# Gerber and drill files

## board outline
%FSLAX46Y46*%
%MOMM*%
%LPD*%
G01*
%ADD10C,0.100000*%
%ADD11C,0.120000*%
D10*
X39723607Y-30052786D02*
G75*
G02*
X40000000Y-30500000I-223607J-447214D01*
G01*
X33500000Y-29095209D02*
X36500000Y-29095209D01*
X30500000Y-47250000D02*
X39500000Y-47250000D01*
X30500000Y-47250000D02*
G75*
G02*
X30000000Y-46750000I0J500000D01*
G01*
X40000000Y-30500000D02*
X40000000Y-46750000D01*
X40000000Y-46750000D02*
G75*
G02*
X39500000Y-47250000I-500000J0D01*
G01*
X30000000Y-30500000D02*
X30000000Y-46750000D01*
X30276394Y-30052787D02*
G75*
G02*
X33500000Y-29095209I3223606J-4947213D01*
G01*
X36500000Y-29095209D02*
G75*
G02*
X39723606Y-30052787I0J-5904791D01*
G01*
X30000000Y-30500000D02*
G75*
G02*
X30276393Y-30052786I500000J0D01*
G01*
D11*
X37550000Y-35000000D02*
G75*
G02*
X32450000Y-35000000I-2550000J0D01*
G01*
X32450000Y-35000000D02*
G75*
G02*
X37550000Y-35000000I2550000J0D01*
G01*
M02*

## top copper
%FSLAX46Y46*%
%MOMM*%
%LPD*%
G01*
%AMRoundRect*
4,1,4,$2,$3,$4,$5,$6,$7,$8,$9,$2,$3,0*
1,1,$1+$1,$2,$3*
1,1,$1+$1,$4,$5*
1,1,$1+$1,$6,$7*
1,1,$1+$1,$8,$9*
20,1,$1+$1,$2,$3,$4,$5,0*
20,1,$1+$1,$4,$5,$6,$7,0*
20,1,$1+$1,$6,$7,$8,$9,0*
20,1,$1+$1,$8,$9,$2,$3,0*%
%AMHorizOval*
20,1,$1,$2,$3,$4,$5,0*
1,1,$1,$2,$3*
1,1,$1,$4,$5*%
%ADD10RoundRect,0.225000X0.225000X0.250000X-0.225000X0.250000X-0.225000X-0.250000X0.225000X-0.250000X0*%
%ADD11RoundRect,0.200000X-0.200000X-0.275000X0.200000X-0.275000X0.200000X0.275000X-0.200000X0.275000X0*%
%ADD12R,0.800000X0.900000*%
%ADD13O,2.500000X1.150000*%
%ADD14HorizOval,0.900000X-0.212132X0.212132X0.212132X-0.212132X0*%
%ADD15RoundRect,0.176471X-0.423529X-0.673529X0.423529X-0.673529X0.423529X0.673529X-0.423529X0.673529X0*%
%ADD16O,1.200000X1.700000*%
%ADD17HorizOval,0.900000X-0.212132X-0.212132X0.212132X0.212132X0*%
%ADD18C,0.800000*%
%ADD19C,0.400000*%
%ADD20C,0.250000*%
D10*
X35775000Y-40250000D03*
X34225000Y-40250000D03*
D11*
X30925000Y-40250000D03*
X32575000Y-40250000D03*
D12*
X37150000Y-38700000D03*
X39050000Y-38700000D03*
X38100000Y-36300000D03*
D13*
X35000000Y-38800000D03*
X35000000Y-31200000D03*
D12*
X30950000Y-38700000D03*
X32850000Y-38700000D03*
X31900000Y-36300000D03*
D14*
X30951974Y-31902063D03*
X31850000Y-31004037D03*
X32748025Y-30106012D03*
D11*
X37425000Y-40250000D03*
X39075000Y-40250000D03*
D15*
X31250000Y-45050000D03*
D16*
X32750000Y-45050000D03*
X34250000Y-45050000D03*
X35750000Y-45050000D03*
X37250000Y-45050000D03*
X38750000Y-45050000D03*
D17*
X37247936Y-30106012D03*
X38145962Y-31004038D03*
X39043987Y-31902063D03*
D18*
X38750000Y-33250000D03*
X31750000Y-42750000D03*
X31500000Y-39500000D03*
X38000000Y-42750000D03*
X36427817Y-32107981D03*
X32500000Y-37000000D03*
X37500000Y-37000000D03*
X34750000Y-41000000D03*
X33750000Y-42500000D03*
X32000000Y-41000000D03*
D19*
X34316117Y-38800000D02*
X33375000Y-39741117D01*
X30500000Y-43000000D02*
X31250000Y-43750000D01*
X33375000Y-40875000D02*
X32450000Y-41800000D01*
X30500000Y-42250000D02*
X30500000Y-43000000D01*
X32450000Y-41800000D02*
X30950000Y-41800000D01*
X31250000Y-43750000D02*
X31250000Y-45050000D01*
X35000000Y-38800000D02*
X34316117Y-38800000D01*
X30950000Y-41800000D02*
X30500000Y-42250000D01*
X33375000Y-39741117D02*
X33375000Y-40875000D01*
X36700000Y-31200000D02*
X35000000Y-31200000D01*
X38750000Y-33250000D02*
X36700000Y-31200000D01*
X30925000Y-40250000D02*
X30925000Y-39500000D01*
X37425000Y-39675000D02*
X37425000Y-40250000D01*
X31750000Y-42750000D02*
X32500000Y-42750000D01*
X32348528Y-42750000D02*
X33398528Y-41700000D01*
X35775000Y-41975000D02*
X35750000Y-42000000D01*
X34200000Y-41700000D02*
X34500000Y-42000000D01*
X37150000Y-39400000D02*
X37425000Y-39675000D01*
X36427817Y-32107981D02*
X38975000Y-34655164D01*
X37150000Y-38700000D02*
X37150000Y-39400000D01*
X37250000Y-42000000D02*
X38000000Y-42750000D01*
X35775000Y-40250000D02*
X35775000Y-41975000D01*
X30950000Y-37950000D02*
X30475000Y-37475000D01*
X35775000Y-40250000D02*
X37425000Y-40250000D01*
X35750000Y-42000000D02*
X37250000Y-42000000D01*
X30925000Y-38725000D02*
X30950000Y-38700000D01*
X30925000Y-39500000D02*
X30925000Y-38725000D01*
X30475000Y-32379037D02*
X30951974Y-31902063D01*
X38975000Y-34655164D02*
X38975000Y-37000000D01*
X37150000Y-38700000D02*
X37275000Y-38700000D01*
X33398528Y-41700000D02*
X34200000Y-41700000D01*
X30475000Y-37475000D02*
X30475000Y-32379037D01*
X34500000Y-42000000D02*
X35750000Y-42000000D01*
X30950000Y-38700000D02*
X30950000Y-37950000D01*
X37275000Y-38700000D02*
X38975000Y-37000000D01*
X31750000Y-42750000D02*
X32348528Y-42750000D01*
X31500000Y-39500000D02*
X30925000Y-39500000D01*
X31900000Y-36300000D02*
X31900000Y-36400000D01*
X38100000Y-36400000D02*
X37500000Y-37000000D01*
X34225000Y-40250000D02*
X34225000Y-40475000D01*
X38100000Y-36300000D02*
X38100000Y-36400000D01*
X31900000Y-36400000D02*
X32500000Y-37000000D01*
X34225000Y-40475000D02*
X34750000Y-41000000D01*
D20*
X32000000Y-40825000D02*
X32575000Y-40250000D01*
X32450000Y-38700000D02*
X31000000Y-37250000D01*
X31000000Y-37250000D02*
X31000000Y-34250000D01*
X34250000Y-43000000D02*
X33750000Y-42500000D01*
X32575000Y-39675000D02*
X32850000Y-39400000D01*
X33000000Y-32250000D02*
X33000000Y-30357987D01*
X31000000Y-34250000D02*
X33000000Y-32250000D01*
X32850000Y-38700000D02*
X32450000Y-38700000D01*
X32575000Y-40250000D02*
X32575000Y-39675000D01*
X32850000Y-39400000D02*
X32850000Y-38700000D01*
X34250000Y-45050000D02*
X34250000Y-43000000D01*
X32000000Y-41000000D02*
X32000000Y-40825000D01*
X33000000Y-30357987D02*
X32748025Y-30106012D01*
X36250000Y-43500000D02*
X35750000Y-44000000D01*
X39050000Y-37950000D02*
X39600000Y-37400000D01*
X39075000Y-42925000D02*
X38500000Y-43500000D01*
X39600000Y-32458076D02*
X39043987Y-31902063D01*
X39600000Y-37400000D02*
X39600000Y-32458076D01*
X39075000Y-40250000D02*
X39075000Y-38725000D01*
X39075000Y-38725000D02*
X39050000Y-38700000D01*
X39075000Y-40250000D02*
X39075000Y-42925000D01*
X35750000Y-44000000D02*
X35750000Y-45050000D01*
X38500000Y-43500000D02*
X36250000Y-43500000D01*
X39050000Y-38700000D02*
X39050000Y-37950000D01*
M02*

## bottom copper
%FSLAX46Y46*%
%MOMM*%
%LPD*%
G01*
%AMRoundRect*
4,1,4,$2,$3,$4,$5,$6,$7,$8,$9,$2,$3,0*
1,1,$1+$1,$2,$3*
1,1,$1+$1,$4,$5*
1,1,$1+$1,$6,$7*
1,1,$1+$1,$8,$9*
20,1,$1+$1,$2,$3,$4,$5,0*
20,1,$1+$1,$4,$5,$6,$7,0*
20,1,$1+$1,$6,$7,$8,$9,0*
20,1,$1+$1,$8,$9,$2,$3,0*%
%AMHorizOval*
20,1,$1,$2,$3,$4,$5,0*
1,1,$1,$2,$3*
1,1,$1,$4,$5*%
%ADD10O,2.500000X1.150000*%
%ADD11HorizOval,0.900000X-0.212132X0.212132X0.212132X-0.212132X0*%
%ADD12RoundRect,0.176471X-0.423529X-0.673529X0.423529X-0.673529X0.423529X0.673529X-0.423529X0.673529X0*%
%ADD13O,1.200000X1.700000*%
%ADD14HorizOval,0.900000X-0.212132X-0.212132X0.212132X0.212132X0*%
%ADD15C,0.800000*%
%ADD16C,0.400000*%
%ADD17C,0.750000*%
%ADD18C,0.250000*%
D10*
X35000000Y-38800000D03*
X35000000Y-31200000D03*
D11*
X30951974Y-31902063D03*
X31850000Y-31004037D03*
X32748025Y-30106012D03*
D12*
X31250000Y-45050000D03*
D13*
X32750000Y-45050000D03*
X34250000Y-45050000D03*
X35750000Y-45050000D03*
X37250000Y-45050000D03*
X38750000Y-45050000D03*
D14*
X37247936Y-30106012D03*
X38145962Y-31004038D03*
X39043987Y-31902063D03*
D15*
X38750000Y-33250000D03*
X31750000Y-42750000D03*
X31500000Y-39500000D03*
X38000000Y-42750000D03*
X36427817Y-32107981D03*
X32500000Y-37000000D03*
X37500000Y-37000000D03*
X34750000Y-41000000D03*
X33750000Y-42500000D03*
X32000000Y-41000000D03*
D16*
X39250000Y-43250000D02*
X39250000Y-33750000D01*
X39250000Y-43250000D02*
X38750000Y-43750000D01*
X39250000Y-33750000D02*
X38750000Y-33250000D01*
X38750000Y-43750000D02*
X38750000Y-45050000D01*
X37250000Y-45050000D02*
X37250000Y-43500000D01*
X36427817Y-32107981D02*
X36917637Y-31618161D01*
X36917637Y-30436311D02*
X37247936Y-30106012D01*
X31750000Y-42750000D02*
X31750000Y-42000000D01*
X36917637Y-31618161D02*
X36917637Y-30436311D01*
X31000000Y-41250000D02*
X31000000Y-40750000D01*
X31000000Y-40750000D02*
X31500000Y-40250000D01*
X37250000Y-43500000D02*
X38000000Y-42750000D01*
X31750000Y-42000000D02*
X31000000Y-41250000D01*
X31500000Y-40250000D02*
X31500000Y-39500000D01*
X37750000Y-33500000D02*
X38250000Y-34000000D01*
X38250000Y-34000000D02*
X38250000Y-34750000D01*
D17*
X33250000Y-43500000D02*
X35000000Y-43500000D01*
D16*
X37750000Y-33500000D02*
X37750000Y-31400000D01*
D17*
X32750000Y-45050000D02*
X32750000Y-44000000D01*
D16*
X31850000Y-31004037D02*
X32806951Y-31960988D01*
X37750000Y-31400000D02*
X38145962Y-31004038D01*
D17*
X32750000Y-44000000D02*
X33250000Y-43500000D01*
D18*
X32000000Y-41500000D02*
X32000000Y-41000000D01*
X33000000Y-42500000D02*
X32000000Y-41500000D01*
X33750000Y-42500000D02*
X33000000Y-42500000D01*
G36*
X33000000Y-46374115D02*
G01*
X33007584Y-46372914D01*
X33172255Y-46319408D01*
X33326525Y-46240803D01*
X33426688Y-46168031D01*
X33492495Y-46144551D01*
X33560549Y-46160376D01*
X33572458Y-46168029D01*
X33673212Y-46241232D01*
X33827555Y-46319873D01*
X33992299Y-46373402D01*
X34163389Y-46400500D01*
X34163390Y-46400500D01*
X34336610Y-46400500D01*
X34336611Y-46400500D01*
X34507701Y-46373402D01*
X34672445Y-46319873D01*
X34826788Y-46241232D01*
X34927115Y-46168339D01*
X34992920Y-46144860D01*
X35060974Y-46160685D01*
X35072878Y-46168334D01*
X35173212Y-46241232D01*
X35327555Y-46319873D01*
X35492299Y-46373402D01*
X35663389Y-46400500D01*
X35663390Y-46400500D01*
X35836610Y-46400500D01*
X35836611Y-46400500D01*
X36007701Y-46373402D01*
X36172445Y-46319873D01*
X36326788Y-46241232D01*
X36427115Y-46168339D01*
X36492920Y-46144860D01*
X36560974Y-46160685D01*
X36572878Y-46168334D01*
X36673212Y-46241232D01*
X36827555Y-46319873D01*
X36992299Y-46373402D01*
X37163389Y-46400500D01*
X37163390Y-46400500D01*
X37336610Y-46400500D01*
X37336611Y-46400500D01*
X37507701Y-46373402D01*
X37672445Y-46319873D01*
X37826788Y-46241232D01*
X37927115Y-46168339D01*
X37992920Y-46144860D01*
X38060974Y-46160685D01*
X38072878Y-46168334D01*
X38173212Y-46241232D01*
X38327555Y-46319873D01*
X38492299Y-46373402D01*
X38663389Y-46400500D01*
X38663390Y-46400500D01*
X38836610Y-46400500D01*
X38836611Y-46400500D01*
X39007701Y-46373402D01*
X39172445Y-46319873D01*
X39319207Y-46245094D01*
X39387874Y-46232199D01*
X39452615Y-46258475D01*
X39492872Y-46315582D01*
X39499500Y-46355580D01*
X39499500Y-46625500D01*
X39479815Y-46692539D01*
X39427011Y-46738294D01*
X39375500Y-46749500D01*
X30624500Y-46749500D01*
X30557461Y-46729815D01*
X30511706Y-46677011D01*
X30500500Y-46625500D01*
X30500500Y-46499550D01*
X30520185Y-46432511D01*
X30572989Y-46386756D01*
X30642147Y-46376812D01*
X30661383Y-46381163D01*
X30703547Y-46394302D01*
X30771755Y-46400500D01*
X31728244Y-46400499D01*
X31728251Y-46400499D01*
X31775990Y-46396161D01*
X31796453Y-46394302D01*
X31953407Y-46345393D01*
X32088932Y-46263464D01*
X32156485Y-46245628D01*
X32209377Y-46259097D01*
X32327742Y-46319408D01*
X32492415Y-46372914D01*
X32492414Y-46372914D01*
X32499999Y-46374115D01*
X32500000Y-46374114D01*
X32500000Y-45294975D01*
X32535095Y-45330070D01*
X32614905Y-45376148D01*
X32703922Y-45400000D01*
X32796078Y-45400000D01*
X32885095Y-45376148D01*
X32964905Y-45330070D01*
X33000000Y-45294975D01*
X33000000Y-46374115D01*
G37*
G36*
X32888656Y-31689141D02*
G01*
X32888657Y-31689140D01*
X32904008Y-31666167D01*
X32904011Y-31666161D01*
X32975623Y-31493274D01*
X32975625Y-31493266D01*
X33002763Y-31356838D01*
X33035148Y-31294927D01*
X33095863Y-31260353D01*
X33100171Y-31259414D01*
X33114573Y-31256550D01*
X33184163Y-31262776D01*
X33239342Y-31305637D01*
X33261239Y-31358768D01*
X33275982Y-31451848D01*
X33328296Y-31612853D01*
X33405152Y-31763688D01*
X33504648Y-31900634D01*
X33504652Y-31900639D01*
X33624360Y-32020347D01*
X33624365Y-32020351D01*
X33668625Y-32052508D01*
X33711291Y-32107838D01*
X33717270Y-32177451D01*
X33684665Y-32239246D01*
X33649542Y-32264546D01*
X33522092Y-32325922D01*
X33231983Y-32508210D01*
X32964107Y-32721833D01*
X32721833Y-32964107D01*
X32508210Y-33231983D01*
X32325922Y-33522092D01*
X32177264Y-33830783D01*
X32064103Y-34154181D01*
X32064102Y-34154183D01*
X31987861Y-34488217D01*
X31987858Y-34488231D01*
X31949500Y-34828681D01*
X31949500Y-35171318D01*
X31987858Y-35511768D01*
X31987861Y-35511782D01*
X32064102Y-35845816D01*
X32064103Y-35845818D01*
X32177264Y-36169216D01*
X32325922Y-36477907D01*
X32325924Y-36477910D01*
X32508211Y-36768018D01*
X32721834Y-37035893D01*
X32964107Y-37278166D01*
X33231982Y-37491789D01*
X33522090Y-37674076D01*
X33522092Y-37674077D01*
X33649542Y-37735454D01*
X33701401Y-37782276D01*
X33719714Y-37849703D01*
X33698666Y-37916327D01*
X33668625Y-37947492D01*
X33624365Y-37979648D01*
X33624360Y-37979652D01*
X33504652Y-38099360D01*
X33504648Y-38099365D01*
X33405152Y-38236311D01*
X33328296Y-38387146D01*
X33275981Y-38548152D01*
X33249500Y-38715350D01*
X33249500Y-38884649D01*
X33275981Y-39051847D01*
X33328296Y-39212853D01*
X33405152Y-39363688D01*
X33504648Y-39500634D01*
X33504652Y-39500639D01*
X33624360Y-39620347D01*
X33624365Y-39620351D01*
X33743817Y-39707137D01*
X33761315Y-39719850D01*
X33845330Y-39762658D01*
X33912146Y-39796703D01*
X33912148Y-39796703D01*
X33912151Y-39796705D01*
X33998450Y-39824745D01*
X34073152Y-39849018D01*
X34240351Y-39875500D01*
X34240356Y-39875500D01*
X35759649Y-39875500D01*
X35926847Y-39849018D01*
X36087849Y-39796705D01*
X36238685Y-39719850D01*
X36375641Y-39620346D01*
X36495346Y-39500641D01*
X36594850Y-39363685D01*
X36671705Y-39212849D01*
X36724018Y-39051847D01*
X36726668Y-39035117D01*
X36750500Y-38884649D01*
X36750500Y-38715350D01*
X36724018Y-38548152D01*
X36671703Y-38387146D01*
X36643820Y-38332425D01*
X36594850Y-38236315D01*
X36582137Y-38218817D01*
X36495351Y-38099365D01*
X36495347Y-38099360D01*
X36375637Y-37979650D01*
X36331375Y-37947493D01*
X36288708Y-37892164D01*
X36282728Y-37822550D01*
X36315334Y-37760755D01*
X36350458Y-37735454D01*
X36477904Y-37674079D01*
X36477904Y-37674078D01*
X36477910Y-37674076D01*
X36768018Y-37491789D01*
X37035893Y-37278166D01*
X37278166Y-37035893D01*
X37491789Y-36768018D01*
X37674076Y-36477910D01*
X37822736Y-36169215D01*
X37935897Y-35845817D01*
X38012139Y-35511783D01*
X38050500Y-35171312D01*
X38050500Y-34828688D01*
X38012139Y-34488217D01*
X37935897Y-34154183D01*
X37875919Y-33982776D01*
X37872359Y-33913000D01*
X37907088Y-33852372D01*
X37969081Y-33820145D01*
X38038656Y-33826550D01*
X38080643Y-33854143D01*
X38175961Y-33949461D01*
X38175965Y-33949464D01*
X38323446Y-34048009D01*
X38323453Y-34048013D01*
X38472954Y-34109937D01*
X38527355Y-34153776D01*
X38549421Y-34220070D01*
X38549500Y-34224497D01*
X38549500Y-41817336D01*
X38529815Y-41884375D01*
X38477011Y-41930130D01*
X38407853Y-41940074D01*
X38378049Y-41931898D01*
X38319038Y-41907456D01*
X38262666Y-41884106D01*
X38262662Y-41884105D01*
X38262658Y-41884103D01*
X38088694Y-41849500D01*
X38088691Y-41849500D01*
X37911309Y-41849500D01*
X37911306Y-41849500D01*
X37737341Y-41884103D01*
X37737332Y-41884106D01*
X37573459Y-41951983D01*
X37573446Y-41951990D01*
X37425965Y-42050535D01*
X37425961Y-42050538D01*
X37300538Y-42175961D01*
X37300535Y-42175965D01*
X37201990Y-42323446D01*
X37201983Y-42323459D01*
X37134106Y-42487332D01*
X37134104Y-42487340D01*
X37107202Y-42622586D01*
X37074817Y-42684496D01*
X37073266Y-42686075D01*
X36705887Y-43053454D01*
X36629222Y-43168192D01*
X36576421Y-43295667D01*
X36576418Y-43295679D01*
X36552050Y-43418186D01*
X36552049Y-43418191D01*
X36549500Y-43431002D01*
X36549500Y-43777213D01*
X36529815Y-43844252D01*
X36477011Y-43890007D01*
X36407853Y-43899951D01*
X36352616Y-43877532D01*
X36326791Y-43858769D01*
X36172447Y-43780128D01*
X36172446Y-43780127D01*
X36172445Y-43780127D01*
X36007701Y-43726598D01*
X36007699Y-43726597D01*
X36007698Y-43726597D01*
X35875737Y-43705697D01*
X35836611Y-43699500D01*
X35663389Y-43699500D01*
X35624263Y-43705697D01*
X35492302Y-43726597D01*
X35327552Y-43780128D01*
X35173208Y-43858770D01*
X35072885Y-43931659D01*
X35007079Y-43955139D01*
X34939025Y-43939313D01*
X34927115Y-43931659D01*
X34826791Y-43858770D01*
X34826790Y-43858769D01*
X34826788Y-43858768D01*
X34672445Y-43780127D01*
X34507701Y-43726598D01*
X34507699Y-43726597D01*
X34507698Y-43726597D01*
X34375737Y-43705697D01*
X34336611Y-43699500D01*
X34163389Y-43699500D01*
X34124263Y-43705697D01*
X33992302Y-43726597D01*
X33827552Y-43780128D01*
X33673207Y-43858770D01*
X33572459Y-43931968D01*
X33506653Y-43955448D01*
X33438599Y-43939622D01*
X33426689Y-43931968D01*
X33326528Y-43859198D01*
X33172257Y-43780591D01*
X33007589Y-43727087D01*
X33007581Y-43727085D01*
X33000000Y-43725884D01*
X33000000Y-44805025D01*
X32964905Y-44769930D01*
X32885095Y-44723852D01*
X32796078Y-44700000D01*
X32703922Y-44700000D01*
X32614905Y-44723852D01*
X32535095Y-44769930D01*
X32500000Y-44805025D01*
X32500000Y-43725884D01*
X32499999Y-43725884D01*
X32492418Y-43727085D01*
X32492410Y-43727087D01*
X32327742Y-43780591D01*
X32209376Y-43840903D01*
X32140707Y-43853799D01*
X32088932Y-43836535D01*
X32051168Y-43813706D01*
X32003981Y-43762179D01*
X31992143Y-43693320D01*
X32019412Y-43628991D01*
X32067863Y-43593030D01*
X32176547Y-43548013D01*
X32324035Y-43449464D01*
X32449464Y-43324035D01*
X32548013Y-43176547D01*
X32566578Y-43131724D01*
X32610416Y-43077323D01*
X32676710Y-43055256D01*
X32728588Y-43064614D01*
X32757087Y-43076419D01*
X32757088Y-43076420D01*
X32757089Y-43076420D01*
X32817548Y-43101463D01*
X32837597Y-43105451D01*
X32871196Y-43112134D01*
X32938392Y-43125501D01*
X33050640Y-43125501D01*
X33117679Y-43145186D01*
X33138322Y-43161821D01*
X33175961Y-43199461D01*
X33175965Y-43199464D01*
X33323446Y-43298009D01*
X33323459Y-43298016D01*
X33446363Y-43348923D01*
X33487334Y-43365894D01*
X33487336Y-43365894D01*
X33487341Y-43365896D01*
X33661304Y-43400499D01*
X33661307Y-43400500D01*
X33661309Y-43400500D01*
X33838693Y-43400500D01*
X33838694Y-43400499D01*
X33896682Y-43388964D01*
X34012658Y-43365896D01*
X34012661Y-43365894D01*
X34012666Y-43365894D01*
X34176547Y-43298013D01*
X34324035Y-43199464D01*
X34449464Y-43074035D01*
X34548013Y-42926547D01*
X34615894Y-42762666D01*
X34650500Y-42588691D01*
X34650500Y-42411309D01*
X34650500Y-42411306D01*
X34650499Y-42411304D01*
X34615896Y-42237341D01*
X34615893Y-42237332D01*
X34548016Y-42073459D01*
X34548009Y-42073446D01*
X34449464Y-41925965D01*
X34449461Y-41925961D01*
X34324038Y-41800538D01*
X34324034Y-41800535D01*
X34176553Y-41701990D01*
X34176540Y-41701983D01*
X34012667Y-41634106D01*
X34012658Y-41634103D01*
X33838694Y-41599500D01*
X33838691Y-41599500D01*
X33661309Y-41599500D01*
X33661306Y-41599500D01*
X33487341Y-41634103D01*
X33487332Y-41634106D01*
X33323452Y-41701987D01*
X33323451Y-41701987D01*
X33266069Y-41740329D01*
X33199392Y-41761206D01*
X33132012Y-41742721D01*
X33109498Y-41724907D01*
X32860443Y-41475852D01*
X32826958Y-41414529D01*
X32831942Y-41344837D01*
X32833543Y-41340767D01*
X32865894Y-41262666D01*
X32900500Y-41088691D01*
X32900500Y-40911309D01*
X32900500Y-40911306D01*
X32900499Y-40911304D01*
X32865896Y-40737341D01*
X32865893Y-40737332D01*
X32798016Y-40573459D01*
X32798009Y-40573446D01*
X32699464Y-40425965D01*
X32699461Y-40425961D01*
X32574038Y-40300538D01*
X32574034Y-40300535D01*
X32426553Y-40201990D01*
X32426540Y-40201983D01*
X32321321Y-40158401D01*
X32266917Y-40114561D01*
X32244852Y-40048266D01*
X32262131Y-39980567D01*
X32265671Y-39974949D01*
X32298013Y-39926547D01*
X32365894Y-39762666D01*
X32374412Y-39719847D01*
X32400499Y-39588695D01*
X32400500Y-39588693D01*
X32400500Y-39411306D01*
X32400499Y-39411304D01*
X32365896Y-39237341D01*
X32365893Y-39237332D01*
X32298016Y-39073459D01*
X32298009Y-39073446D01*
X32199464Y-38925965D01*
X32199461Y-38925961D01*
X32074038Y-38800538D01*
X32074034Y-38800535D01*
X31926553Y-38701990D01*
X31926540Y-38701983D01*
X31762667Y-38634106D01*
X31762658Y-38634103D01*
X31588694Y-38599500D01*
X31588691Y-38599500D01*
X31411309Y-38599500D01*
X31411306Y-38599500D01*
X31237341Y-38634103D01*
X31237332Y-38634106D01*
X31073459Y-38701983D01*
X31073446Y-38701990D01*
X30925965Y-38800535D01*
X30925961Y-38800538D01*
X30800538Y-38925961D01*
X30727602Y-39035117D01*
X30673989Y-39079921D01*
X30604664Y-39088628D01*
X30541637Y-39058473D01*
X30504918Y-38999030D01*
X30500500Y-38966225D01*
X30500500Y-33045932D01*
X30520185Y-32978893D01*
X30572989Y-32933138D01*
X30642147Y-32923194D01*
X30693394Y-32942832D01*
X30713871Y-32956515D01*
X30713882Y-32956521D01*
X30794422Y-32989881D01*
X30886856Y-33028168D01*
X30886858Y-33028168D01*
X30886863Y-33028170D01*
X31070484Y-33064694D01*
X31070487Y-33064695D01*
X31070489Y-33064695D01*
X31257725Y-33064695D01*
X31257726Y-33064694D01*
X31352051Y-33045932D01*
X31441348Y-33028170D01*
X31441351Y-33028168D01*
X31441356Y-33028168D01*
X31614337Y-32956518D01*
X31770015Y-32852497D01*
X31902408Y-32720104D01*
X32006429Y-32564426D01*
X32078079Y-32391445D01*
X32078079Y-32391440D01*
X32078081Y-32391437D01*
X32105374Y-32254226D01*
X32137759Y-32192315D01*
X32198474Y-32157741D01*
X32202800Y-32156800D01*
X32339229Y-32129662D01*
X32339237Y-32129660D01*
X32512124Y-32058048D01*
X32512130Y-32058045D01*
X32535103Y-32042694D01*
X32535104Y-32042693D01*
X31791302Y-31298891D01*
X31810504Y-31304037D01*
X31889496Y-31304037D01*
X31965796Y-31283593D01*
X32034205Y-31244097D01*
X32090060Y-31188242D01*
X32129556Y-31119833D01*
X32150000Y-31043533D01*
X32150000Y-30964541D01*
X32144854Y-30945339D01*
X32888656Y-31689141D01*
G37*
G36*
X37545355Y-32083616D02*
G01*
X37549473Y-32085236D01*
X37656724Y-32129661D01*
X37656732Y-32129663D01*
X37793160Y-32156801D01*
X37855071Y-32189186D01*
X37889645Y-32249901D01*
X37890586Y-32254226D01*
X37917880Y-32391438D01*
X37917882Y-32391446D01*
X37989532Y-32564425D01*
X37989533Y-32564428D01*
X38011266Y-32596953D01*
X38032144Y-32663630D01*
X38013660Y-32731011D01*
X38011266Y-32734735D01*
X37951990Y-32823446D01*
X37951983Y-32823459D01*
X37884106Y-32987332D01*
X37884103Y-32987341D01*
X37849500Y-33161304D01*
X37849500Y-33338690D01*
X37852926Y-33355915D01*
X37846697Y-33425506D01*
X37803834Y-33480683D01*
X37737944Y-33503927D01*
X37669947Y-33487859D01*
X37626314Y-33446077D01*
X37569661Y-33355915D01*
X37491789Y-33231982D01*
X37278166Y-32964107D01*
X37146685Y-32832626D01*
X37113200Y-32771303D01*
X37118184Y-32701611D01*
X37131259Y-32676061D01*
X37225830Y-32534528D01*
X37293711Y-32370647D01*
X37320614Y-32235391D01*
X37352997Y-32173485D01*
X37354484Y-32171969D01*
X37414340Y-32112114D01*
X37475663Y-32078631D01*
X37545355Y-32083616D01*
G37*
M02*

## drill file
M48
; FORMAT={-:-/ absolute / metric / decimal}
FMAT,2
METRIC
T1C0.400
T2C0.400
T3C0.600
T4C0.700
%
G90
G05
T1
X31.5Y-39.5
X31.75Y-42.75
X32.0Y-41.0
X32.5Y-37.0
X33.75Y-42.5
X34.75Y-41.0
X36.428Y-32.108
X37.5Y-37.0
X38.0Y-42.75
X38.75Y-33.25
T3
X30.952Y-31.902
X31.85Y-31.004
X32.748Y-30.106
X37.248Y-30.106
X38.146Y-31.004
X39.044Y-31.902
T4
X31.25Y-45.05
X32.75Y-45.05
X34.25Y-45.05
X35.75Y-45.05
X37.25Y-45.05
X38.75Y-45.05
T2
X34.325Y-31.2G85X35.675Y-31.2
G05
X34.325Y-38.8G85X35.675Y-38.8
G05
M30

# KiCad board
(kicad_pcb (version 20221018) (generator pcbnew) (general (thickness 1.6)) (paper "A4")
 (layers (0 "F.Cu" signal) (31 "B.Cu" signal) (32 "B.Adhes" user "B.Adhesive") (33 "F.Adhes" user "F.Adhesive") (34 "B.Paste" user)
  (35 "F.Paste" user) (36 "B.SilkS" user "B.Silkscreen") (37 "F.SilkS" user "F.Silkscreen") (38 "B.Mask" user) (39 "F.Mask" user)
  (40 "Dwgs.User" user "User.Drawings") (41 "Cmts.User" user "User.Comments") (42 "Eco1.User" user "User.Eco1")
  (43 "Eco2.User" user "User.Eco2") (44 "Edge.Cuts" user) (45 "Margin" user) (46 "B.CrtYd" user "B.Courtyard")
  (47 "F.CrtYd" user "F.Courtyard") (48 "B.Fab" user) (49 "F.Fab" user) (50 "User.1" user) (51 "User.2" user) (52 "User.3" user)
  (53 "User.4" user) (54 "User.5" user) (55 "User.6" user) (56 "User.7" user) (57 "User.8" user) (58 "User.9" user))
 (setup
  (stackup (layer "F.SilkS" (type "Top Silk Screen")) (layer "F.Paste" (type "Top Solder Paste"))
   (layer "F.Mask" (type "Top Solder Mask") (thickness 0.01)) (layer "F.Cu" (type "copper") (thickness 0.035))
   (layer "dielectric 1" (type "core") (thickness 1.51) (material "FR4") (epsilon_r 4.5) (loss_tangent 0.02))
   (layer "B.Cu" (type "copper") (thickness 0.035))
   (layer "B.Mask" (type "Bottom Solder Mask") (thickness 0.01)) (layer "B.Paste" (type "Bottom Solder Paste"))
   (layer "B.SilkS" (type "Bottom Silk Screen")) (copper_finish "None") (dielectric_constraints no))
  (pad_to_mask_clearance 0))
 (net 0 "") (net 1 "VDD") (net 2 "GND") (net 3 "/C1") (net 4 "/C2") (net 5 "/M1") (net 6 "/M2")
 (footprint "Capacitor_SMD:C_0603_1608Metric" (layer "F.Cu") (at 35 40.25 180)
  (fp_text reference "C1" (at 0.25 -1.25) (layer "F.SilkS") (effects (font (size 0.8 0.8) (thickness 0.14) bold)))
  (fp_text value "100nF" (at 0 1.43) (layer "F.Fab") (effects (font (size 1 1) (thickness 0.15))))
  (pad "1" smd roundrect (at -0.775 0 180) (size 0.9 0.95) (layers "F.Cu" "F.Paste" "F.Mask") (roundrect_rratio 0.25) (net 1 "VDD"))
  (pad "2" smd roundrect (at 0.775 0 180) (size 0.9 0.95) (layers "F.Cu" "F.Paste" "F.Mask") (roundrect_rratio 0.25) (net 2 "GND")))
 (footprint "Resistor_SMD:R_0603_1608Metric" (layer "F.Cu") (at 31.75 40.25)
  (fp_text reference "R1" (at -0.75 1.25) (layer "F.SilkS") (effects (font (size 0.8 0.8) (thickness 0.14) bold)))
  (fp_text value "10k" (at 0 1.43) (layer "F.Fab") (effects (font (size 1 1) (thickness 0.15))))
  (pad "1" smd roundrect (at -0.825 0) (size 0.8 0.95) (layers "F.Cu" "F.Paste" "F.Mask") (roundrect_rratio 0.25) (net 1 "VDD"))
  (pad "2" smd roundrect (at 0.825 0) (size 0.8 0.95) (layers "F.Cu" "F.Paste" "F.Mask") (roundrect_rratio 0.25) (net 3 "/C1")))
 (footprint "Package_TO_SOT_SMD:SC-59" (layer "F.Cu") (at 38.1 37.5 90)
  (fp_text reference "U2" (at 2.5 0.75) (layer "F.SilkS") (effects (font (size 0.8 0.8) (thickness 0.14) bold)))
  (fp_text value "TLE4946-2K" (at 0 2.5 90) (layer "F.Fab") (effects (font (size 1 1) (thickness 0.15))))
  (pad "1" smd rect (at -1.2 -0.95 90) (size 0.9 0.8) (layers "F.Cu" "F.Paste" "F.Mask") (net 1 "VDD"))
  (pad "2" smd rect (at -1.2 0.95 90) (size 0.9 0.8) (layers "F.Cu" "F.Paste" "F.Mask") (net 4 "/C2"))
  (pad "3" smd rect (at 1.2 0 90) (size 0.9 0.8) (layers "F.Cu" "F.Paste" "F.Mask") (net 2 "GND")))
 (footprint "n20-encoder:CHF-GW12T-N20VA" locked (layer "F.Cu") (at 35 35 90)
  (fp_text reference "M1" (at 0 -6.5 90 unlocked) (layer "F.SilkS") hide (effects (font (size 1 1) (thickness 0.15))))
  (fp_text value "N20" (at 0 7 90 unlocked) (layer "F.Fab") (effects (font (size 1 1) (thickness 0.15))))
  (fp_circle (center 0 0) (end 2.55 0) (stroke (width 0.12) (type default)) (fill none) (layer "Edge.Cuts"))
  (pad "1" thru_hole oval locked (at -3.8 0 90) (size 1.15 2.5) (drill oval 0.4 1.75) (layers "*.Cu" "*.Mask") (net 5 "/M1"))
  (pad "2" thru_hole oval locked (at 3.8 0 90) (size 1.15 2.5) (drill oval 0.4 1.75) (layers "*.Cu" "*.Mask") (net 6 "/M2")))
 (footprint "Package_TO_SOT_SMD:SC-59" (layer "F.Cu") (at 31.9 37.5 90)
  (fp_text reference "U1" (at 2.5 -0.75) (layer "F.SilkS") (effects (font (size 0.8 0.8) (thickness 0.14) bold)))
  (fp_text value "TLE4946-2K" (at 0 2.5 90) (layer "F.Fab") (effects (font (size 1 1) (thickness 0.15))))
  (pad "1" smd rect (at -1.2 -0.95 90) (size 0.9 0.8) (layers "F.Cu" "F.Paste" "F.Mask") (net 1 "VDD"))
  (pad "2" smd rect (at -1.2 0.95 90) (size 0.9 0.8) (layers "F.Cu" "F.Paste" "F.Mask") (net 3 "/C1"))
  (pad "3" smd rect (at 1.2 0 90) (size 0.9 0.8) (layers "F.Cu" "F.Paste" "F.Mask") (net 2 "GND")))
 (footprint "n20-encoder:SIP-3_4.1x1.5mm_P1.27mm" (layer "F.Cu") (at 30.951974 31.902063 45)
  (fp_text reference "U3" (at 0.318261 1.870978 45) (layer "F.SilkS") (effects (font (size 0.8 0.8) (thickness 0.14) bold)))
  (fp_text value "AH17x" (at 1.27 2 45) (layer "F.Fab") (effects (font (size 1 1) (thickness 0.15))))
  (pad "1" thru_hole oval (at 0 0 45) (size 0.9 1.5) (drill 0.6) (layers "*.Cu" "*.Mask") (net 1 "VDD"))
  (pad "2" thru_hole oval (at 1.27 0 45) (size 0.9 1.5) (drill 0.6) (layers "*.Cu" "*.Mask") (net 2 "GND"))
  (pad "3" thru_hole oval (at 2.54 0 45) (size 0.9 1.5) (drill 0.6) (layers "*.Cu" "*.Mask") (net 3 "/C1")))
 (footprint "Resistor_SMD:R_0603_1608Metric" (layer "F.Cu") (at 38.25 40.25)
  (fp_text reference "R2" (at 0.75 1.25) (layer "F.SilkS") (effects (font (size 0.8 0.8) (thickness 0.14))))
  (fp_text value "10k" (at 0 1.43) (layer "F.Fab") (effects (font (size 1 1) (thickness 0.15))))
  (pad "1" smd roundrect (at -0.825 0) (size 0.8 0.95) (layers "F.Cu" "F.Paste" "F.Mask") (roundrect_rratio 0.25) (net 1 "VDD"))
  (pad "2" smd roundrect (at 0.825 0) (size 0.8 0.95) (layers "F.Cu" "F.Paste" "F.Mask") (roundrect_rratio 0.25) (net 4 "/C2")))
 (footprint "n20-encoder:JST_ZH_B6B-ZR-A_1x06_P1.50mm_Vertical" (layer "F.Cu") (at 31.25 45.05)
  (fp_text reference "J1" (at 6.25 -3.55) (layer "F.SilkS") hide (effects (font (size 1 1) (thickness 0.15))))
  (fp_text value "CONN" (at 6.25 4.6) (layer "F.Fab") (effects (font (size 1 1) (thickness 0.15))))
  (pad "1" thru_hole roundrect (at 0 0) (size 1.2 1.7) (drill 0.7) (layers "*.Cu" "*.Mask") (roundrect_rratio 0.147059) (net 5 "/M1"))
  (pad "2" thru_hole oval (at 1.5 0) (size 1.2 1.7) (drill 0.7) (layers "*.Cu" "*.Mask") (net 2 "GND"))
  (pad "3" thru_hole oval (at 3 0) (size 1.2 1.7) (drill 0.7) (layers "*.Cu" "*.Mask") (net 3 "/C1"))
  (pad "4" thru_hole oval (at 4.5 0) (size 1.2 1.7) (drill 0.7) (layers "*.Cu" "*.Mask") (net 4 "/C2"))
  (pad "5" thru_hole oval (at 6 0) (size 1.2 1.7) (drill 0.7) (layers "*.Cu" "*.Mask") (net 1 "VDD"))
  (pad "6" thru_hole oval (at 7.5 0) (size 1.2 1.7) (drill 0.7) (layers "*.Cu" "*.Mask") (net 6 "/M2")))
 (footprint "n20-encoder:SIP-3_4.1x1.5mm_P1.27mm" (layer "F.Cu") (at 37.247936 30.106012 -45)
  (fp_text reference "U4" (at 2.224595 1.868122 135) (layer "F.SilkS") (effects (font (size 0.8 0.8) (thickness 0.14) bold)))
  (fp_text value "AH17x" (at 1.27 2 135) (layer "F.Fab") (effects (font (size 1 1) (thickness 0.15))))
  (pad "1" thru_hole oval (at 0 0 315) (size 0.9 1.5) (drill 0.6) (layers "*.Cu" "*.Mask") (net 1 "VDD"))
  (pad "2" thru_hole oval (at 1.27 0 315) (size 0.9 1.5) (drill 0.6) (layers "*.Cu" "*.Mask") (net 2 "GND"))
  (pad "3" thru_hole oval (at 2.54 0 315) (size 0.9 1.5) (drill 0.6) (layers "*.Cu" "*.Mask") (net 4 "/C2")))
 (gr_arc (start 39.723607 30.052786) (mid 39.925326 30.237134) (end 40 30.5) (stroke (width 0.1) (type default)) (layer "Edge.Cuts"))
 (gr_line (start 33.5 29.095209) (end 36.5 29.095209) (stroke (width 0.1) (type default)) (layer "Edge.Cuts"))
 (gr_line (start 30.5 47.25) (end 39.5 47.25) (stroke (width 0.1) (type default)) (layer "Edge.Cuts"))
 (gr_arc (start 30.5 47.25) (mid 30.146447 47.103553) (end 30 46.75) (stroke (width 0.1) (type default)) (layer "Edge.Cuts"))
 (gr_line (start 40 30.5) (end 40 46.75) (stroke (width 0.1) (type default)) (layer "Edge.Cuts"))
 (gr_arc (start 40 46.75) (mid 39.853553 47.103553) (end 39.5 47.25) (stroke (width 0.1) (type default)) (layer "Edge.Cuts"))
 (gr_line (start 30 30.5) (end 30 46.75) (stroke (width 0.1) (type default)) (layer "Edge.Cuts"))
 (gr_arc (start 30.276394 30.052787) (mid 31.818588 29.339664) (end 33.5 29.095209) (stroke (width 0.1) (type default)) (layer "Edge.Cuts"))
 (gr_arc (start 36.5 29.095209) (mid 38.181413 29.339664) (end 39.723606 30.052787) (stroke (width 0.1) (type default)) (layer "Edge.Cuts"))
 (gr_arc (start 30 30.5) (mid 30.074675 30.237134) (end 30.276393 30.052786) (stroke (width 0.1) (type default)) (layer "Edge.Cuts"))
 (segment (start 34.316117 38.8) (end 33.375 39.741117) (width 0.4) (layer "F.Cu") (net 5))
 (segment (start 30.5 43) (end 31.25 43.75) (width 0.4) (layer "F.Cu") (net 5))
 (segment (start 33.375 40.875) (end 32.45 41.8) (width 0.4) (layer "F.Cu") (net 5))
 (segment (start 30.5 42.25) (end 30.5 43) (width 0.4) (layer "F.Cu") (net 5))
 (segment (start 32.45 41.8) (end 30.95 41.8) (width 0.4) (layer "F.Cu") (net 5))
 (segment (start 31.25 43.75) (end 31.25 45.05) (width 0.4) (layer "F.Cu") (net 5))
 (segment (start 35 38.8) (end 34.316117 38.8) (width 0.4) (layer "F.Cu") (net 5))
 (segment (start 30.95 41.8) (end 30.5 42.25) (width 0.4) (layer "F.Cu") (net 5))
 (segment (start 33.375 39.741117) (end 33.375 40.875) (width 0.4) (layer "F.Cu") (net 5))
 (segment (start 36.7 31.2) (end 35 31.2) (width 0.4) (layer "F.Cu") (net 6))
 (segment (start 38.75 33.25) (end 36.7 31.2) (width 0.4) (layer "F.Cu") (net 6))
 (via (at 38.75 33.25) (size 0.8) (drill 0.4) (layers "F.Cu" "B.Cu") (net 6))
 (segment (start 39.25 43.25) (end 39.25 33.75) (width 0.4) (layer "B.Cu") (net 6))
 (segment (start 39.25 43.25) (end 38.75 43.75) (width 0.4) (layer "B.Cu") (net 6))
 (segment (start 39.25 33.75) (end 38.75 33.25) (width 0.4) (layer "B.Cu") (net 6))
 (segment (start 38.75 43.75) (end 38.75 45.05) (width 0.4) (layer "B.Cu") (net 6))
 (segment (start 30.925 40.25) (end 30.925 39.5) (width 0.4) (layer "F.Cu") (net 1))
 (segment (start 37.425 39.675) (end 37.425 40.25) (width 0.4) (layer "F.Cu") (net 1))
 (segment (start 31.75 42.75) (end 32.5 42.75) (width 0.4) (layer "F.Cu") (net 1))
 (segment (start 32.348528 42.75) (end 33.398528 41.7) (width 0.4) (layer "F.Cu") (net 1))
 (segment (start 35.775 41.975) (end 35.75 42) (width 0.4) (layer "F.Cu") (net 1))
 (segment (start 34.2 41.7) (end 34.5 42) (width 0.4) (layer "F.Cu") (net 1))
 (segment (start 37.15 39.4) (end 37.425 39.675) (width 0.4) (layer "F.Cu") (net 1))
 (segment (start 36.427817 32.107981) (end 38.975 34.655164) (width 0.4) (layer "F.Cu") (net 1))
 (segment (start 37.15 38.7) (end 37.15 39.4) (width 0.4) (layer "F.Cu") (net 1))
 (segment (start 37.25 42) (end 38 42.75) (width 0.4) (layer "F.Cu") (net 1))
 (segment (start 35.775 40.25) (end 35.775 41.975) (width 0.4) (layer "F.Cu") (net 1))
 (segment (start 30.95 37.95) (end 30.475 37.475) (width 0.4) (layer "F.Cu") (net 1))
 (segment (start 35.775 40.25) (end 37.425 40.25) (width 0.4) (layer "F.Cu") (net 1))
 (segment (start 35.75 42) (end 37.25 42) (width 0.4) (layer "F.Cu") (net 1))
 (segment (start 30.925 38.725) (end 30.95 38.7) (width 0.4) (layer "F.Cu") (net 1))
 (segment (start 30.925 39.5) (end 30.925 38.725) (width 0.4) (layer "F.Cu") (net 1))
 (segment (start 30.475 32.379037) (end 30.951974 31.902063) (width 0.4) (layer "F.Cu") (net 1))
 (segment (start 38.975 34.655164) (end 38.975 37) (width 0.4) (layer "F.Cu") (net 1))
 (segment (start 37.15 38.7) (end 37.275 38.7) (width 0.4) (layer "F.Cu") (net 1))
 (segment (start 33.398528 41.7) (end 34.2 41.7) (width 0.4) (layer "F.Cu") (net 1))
 (segment (start 30.475 37.475) (end 30.475 32.379037) (width 0.4) (layer "F.Cu") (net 1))
 (segment (start 34.5 42) (end 35.75 42) (width 0.4) (layer "F.Cu") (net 1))
 (segment (start 30.95 38.7) (end 30.95 37.95) (width 0.4) (layer "F.Cu") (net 1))
 (segment (start 37.275 38.7) (end 38.975 37) (width 0.4) (layer "F.Cu") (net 1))
 (segment (start 31.75 42.75) (end 32.348528 42.75) (width 0.4) (layer "F.Cu") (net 1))
 (segment (start 31.5 39.5) (end 30.925 39.5) (width 0.4) (layer "F.Cu") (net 1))
 (via (at 31.75 42.75) (size 0.8) (drill 0.4) (layers "F.Cu" "B.Cu") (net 1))
 (via (at 31.5 39.5) (size 0.8) (drill 0.4) (layers "F.Cu" "B.Cu") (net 1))
 (via (at 38 42.75) (size 0.8) (drill 0.4) (layers "F.Cu" "B.Cu") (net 1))
 (via (at 36.427817 32.107981) (size 0.8) (drill 0.4) (layers "F.Cu" "B.Cu") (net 1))
 (segment (start 37.25 45.05) (end 37.25 43.5) (width 0.4) (layer "B.Cu") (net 1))
 (segment (start 36.427817 32.107981) (end 36.917637 31.618161) (width 0.4) (layer "B.Cu") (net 1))
 (segment (start 36.917637 30.436311) (end 37.247936 30.106012) (width 0.4) (layer "B.Cu") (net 1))
 (segment (start 31.75 42.75) (end 31.75 42) (width 0.4) (layer "B.Cu") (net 1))
 (segment (start 36.917637 31.618161) (end 36.917637 30.436311) (width 0.4) (layer "B.Cu") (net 1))
 (segment (start 31 41.25) (end 31 40.75) (width 0.4) (layer "B.Cu") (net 1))
 (segment (start 31 40.75) (end 31.5 40.25) (width 0.4) (layer "B.Cu") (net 1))
 (segment (start 37.25 43.5) (end 38 42.75) (width 0.4) (layer "B.Cu") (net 1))
 (segment (start 31.75 42) (end 31 41.25) (width 0.4) (layer "B.Cu") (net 1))
 (segment (start 31.5 40.25) (end 31.5 39.5) (width 0.4) (layer "B.Cu") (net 1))
 (segment (start 31.9 36.3) (end 31.9 36.4) (width 0.4) (layer "F.Cu") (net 2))
 (segment (start 38.1 36.4) (end 37.5 37) (width 0.4) (layer "F.Cu") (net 2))
 (segment (start 34.225 40.25) (end 34.225 40.475) (width 0.4) (layer "F.Cu") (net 2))
 (segment (start 38.1 36.3) (end 38.1 36.4) (width 0.4) (layer "F.Cu") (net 2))
 (segment (start 31.9 36.4) (end 32.5 37) (width 0.4) (layer "F.Cu") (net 2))
 (segment (start 34.225 40.475) (end 34.75 41) (width 0.4) (layer "F.Cu") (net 2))
 (via (at 32.5 37) (size 0.8) (drill 0.4) (layers "F.Cu" "B.Cu") (free) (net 2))
 (via (at 37.5 37) (size 0.8) (drill 0.4) (layers "F.Cu" "B.Cu") (free) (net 2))
 (via (at 34.75 41) (size 0.8) (drill 0.4) (layers "F.Cu" "B.Cu") (free) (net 2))
 (segment (start 37.75 33.5) (end 38.25 34) (width 0.4) (layer "B.Cu") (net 2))
 (segment (start 38.25 34) (end 38.25 34.75) (width 0.4) (layer "B.Cu") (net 2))
 (segment (start 33.25 43.5) (end 35 43.5) (width 0.75) (layer "B.Cu") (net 2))
 (segment (start 37.75 33.5) (end 37.75 31.4) (width 0.4) (layer "B.Cu") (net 2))
 (segment (start 32.75 45.05) (end 32.75 44) (width 0.75) (layer "B.Cu") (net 2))
 (segment (start 31.85 31.004037) (end 32.806951 31.960988) (width 0.4) (layer "B.Cu") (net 2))
 (segment (start 37.75 31.4) (end 38.145962 31.004038) (width 0.4) (layer "B.Cu") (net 2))
 (segment (start 32.75 44) (end 33.25 43.5) (width 0.75) (layer "B.Cu") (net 2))
 (segment (start 32 40.825) (end 32.575 40.25) (width 0.25) (layer "F.Cu") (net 3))
 (segment (start 32.45 38.7) (end 31 37.25) (width 0.25) (layer "F.Cu") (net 3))
 (segment (start 31 37.25) (end 31 34.25) (width 0.25) (layer "F.Cu") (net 3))
 (segment (start 34.25 43) (end 33.75 42.5) (width 0.25) (layer "F.Cu") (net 3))
 (segment (start 32.575 39.675) (end 32.85 39.4) (width 0.25) (layer "F.Cu") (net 3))
 (segment (start 33 32.25) (end 33 30.357987) (width 0.25) (layer "F.Cu") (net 3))
 (segment (start 31 34.25) (end 33 32.25) (width 0.25) (layer "F.Cu") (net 3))
 (segment (start 32.85 38.7) (end 32.45 38.7) (width 0.25) (layer "F.Cu") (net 3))
 (segment (start 32.575 40.25) (end 32.575 39.675) (width 0.25) (layer "F.Cu") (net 3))
 (segment (start 32.85 39.4) (end 32.85 38.7) (width 0.25) (layer "F.Cu") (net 3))
 (segment (start 34.25 45.05) (end 34.25 43) (width 0.25) (layer "F.Cu") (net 3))
 (segment (start 32 41) (end 32 40.825) (width 0.25) (layer "F.Cu") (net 3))
 (segment (start 33 30.357987) (end 32.748025 30.106012) (width 0.25) (layer "F.Cu") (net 3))
 (via (at 33.75 42.5) (size 0.8) (drill 0.4) (layers "F.Cu" "B.Cu") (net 3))
 (via (at 32 41) (size 0.8) (drill 0.4) (layers "F.Cu" "B.Cu") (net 3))
 (segment (start 32 41.5) (end 32 41) (width 0.25) (layer "B.Cu") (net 3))
 (segment (start 33 42.5) (end 32 41.5) (width 0.25) (layer "B.Cu") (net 3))
 (segment (start 33.75 42.5) (end 33 42.5) (width 0.25) (layer "B.Cu") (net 3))
 (segment (start 36.25 43.5) (end 35.75 44) (width 0.25) (layer "F.Cu") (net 4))
 (segment (start 39.05 37.95) (end 39.6 37.4) (width 0.25) (layer "F.Cu") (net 4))
 (segment (start 39.075 42.925) (end 38.5 43.5) (width 0.25) (layer "F.Cu") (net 4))
 (segment (start 39.6 32.458076) (end 39.043987 31.902063) (width 0.25) (layer "F.Cu") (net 4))
 (segment (start 39.6 37.4) (end 39.6 32.458076) (width 0.25) (layer "F.Cu") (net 4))
 (segment (start 39.075 40.25) (end 39.075 38.725) (width 0.25) (layer "F.Cu") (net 4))
 (segment (start 39.075 38.725) (end 39.05 38.7) (width 0.25) (layer "F.Cu") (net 4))
 (segment (start 39.075 40.25) (end 39.075 42.925) (width 0.25) (layer "F.Cu") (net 4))
 (segment (start 35.75 44) (end 35.75 45.05) (width 0.25) (layer "F.Cu") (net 4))
 (segment (start 38.5 43.5) (end 36.25 43.5) (width 0.25) (layer "F.Cu") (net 4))
 (segment (start 39.05 38.7) (end 39.05 37.95) (width 0.25) (layer "F.Cu") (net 4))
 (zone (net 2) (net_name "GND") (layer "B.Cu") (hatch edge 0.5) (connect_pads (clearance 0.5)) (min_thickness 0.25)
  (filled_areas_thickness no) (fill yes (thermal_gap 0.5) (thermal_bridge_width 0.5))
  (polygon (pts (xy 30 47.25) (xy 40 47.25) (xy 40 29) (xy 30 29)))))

